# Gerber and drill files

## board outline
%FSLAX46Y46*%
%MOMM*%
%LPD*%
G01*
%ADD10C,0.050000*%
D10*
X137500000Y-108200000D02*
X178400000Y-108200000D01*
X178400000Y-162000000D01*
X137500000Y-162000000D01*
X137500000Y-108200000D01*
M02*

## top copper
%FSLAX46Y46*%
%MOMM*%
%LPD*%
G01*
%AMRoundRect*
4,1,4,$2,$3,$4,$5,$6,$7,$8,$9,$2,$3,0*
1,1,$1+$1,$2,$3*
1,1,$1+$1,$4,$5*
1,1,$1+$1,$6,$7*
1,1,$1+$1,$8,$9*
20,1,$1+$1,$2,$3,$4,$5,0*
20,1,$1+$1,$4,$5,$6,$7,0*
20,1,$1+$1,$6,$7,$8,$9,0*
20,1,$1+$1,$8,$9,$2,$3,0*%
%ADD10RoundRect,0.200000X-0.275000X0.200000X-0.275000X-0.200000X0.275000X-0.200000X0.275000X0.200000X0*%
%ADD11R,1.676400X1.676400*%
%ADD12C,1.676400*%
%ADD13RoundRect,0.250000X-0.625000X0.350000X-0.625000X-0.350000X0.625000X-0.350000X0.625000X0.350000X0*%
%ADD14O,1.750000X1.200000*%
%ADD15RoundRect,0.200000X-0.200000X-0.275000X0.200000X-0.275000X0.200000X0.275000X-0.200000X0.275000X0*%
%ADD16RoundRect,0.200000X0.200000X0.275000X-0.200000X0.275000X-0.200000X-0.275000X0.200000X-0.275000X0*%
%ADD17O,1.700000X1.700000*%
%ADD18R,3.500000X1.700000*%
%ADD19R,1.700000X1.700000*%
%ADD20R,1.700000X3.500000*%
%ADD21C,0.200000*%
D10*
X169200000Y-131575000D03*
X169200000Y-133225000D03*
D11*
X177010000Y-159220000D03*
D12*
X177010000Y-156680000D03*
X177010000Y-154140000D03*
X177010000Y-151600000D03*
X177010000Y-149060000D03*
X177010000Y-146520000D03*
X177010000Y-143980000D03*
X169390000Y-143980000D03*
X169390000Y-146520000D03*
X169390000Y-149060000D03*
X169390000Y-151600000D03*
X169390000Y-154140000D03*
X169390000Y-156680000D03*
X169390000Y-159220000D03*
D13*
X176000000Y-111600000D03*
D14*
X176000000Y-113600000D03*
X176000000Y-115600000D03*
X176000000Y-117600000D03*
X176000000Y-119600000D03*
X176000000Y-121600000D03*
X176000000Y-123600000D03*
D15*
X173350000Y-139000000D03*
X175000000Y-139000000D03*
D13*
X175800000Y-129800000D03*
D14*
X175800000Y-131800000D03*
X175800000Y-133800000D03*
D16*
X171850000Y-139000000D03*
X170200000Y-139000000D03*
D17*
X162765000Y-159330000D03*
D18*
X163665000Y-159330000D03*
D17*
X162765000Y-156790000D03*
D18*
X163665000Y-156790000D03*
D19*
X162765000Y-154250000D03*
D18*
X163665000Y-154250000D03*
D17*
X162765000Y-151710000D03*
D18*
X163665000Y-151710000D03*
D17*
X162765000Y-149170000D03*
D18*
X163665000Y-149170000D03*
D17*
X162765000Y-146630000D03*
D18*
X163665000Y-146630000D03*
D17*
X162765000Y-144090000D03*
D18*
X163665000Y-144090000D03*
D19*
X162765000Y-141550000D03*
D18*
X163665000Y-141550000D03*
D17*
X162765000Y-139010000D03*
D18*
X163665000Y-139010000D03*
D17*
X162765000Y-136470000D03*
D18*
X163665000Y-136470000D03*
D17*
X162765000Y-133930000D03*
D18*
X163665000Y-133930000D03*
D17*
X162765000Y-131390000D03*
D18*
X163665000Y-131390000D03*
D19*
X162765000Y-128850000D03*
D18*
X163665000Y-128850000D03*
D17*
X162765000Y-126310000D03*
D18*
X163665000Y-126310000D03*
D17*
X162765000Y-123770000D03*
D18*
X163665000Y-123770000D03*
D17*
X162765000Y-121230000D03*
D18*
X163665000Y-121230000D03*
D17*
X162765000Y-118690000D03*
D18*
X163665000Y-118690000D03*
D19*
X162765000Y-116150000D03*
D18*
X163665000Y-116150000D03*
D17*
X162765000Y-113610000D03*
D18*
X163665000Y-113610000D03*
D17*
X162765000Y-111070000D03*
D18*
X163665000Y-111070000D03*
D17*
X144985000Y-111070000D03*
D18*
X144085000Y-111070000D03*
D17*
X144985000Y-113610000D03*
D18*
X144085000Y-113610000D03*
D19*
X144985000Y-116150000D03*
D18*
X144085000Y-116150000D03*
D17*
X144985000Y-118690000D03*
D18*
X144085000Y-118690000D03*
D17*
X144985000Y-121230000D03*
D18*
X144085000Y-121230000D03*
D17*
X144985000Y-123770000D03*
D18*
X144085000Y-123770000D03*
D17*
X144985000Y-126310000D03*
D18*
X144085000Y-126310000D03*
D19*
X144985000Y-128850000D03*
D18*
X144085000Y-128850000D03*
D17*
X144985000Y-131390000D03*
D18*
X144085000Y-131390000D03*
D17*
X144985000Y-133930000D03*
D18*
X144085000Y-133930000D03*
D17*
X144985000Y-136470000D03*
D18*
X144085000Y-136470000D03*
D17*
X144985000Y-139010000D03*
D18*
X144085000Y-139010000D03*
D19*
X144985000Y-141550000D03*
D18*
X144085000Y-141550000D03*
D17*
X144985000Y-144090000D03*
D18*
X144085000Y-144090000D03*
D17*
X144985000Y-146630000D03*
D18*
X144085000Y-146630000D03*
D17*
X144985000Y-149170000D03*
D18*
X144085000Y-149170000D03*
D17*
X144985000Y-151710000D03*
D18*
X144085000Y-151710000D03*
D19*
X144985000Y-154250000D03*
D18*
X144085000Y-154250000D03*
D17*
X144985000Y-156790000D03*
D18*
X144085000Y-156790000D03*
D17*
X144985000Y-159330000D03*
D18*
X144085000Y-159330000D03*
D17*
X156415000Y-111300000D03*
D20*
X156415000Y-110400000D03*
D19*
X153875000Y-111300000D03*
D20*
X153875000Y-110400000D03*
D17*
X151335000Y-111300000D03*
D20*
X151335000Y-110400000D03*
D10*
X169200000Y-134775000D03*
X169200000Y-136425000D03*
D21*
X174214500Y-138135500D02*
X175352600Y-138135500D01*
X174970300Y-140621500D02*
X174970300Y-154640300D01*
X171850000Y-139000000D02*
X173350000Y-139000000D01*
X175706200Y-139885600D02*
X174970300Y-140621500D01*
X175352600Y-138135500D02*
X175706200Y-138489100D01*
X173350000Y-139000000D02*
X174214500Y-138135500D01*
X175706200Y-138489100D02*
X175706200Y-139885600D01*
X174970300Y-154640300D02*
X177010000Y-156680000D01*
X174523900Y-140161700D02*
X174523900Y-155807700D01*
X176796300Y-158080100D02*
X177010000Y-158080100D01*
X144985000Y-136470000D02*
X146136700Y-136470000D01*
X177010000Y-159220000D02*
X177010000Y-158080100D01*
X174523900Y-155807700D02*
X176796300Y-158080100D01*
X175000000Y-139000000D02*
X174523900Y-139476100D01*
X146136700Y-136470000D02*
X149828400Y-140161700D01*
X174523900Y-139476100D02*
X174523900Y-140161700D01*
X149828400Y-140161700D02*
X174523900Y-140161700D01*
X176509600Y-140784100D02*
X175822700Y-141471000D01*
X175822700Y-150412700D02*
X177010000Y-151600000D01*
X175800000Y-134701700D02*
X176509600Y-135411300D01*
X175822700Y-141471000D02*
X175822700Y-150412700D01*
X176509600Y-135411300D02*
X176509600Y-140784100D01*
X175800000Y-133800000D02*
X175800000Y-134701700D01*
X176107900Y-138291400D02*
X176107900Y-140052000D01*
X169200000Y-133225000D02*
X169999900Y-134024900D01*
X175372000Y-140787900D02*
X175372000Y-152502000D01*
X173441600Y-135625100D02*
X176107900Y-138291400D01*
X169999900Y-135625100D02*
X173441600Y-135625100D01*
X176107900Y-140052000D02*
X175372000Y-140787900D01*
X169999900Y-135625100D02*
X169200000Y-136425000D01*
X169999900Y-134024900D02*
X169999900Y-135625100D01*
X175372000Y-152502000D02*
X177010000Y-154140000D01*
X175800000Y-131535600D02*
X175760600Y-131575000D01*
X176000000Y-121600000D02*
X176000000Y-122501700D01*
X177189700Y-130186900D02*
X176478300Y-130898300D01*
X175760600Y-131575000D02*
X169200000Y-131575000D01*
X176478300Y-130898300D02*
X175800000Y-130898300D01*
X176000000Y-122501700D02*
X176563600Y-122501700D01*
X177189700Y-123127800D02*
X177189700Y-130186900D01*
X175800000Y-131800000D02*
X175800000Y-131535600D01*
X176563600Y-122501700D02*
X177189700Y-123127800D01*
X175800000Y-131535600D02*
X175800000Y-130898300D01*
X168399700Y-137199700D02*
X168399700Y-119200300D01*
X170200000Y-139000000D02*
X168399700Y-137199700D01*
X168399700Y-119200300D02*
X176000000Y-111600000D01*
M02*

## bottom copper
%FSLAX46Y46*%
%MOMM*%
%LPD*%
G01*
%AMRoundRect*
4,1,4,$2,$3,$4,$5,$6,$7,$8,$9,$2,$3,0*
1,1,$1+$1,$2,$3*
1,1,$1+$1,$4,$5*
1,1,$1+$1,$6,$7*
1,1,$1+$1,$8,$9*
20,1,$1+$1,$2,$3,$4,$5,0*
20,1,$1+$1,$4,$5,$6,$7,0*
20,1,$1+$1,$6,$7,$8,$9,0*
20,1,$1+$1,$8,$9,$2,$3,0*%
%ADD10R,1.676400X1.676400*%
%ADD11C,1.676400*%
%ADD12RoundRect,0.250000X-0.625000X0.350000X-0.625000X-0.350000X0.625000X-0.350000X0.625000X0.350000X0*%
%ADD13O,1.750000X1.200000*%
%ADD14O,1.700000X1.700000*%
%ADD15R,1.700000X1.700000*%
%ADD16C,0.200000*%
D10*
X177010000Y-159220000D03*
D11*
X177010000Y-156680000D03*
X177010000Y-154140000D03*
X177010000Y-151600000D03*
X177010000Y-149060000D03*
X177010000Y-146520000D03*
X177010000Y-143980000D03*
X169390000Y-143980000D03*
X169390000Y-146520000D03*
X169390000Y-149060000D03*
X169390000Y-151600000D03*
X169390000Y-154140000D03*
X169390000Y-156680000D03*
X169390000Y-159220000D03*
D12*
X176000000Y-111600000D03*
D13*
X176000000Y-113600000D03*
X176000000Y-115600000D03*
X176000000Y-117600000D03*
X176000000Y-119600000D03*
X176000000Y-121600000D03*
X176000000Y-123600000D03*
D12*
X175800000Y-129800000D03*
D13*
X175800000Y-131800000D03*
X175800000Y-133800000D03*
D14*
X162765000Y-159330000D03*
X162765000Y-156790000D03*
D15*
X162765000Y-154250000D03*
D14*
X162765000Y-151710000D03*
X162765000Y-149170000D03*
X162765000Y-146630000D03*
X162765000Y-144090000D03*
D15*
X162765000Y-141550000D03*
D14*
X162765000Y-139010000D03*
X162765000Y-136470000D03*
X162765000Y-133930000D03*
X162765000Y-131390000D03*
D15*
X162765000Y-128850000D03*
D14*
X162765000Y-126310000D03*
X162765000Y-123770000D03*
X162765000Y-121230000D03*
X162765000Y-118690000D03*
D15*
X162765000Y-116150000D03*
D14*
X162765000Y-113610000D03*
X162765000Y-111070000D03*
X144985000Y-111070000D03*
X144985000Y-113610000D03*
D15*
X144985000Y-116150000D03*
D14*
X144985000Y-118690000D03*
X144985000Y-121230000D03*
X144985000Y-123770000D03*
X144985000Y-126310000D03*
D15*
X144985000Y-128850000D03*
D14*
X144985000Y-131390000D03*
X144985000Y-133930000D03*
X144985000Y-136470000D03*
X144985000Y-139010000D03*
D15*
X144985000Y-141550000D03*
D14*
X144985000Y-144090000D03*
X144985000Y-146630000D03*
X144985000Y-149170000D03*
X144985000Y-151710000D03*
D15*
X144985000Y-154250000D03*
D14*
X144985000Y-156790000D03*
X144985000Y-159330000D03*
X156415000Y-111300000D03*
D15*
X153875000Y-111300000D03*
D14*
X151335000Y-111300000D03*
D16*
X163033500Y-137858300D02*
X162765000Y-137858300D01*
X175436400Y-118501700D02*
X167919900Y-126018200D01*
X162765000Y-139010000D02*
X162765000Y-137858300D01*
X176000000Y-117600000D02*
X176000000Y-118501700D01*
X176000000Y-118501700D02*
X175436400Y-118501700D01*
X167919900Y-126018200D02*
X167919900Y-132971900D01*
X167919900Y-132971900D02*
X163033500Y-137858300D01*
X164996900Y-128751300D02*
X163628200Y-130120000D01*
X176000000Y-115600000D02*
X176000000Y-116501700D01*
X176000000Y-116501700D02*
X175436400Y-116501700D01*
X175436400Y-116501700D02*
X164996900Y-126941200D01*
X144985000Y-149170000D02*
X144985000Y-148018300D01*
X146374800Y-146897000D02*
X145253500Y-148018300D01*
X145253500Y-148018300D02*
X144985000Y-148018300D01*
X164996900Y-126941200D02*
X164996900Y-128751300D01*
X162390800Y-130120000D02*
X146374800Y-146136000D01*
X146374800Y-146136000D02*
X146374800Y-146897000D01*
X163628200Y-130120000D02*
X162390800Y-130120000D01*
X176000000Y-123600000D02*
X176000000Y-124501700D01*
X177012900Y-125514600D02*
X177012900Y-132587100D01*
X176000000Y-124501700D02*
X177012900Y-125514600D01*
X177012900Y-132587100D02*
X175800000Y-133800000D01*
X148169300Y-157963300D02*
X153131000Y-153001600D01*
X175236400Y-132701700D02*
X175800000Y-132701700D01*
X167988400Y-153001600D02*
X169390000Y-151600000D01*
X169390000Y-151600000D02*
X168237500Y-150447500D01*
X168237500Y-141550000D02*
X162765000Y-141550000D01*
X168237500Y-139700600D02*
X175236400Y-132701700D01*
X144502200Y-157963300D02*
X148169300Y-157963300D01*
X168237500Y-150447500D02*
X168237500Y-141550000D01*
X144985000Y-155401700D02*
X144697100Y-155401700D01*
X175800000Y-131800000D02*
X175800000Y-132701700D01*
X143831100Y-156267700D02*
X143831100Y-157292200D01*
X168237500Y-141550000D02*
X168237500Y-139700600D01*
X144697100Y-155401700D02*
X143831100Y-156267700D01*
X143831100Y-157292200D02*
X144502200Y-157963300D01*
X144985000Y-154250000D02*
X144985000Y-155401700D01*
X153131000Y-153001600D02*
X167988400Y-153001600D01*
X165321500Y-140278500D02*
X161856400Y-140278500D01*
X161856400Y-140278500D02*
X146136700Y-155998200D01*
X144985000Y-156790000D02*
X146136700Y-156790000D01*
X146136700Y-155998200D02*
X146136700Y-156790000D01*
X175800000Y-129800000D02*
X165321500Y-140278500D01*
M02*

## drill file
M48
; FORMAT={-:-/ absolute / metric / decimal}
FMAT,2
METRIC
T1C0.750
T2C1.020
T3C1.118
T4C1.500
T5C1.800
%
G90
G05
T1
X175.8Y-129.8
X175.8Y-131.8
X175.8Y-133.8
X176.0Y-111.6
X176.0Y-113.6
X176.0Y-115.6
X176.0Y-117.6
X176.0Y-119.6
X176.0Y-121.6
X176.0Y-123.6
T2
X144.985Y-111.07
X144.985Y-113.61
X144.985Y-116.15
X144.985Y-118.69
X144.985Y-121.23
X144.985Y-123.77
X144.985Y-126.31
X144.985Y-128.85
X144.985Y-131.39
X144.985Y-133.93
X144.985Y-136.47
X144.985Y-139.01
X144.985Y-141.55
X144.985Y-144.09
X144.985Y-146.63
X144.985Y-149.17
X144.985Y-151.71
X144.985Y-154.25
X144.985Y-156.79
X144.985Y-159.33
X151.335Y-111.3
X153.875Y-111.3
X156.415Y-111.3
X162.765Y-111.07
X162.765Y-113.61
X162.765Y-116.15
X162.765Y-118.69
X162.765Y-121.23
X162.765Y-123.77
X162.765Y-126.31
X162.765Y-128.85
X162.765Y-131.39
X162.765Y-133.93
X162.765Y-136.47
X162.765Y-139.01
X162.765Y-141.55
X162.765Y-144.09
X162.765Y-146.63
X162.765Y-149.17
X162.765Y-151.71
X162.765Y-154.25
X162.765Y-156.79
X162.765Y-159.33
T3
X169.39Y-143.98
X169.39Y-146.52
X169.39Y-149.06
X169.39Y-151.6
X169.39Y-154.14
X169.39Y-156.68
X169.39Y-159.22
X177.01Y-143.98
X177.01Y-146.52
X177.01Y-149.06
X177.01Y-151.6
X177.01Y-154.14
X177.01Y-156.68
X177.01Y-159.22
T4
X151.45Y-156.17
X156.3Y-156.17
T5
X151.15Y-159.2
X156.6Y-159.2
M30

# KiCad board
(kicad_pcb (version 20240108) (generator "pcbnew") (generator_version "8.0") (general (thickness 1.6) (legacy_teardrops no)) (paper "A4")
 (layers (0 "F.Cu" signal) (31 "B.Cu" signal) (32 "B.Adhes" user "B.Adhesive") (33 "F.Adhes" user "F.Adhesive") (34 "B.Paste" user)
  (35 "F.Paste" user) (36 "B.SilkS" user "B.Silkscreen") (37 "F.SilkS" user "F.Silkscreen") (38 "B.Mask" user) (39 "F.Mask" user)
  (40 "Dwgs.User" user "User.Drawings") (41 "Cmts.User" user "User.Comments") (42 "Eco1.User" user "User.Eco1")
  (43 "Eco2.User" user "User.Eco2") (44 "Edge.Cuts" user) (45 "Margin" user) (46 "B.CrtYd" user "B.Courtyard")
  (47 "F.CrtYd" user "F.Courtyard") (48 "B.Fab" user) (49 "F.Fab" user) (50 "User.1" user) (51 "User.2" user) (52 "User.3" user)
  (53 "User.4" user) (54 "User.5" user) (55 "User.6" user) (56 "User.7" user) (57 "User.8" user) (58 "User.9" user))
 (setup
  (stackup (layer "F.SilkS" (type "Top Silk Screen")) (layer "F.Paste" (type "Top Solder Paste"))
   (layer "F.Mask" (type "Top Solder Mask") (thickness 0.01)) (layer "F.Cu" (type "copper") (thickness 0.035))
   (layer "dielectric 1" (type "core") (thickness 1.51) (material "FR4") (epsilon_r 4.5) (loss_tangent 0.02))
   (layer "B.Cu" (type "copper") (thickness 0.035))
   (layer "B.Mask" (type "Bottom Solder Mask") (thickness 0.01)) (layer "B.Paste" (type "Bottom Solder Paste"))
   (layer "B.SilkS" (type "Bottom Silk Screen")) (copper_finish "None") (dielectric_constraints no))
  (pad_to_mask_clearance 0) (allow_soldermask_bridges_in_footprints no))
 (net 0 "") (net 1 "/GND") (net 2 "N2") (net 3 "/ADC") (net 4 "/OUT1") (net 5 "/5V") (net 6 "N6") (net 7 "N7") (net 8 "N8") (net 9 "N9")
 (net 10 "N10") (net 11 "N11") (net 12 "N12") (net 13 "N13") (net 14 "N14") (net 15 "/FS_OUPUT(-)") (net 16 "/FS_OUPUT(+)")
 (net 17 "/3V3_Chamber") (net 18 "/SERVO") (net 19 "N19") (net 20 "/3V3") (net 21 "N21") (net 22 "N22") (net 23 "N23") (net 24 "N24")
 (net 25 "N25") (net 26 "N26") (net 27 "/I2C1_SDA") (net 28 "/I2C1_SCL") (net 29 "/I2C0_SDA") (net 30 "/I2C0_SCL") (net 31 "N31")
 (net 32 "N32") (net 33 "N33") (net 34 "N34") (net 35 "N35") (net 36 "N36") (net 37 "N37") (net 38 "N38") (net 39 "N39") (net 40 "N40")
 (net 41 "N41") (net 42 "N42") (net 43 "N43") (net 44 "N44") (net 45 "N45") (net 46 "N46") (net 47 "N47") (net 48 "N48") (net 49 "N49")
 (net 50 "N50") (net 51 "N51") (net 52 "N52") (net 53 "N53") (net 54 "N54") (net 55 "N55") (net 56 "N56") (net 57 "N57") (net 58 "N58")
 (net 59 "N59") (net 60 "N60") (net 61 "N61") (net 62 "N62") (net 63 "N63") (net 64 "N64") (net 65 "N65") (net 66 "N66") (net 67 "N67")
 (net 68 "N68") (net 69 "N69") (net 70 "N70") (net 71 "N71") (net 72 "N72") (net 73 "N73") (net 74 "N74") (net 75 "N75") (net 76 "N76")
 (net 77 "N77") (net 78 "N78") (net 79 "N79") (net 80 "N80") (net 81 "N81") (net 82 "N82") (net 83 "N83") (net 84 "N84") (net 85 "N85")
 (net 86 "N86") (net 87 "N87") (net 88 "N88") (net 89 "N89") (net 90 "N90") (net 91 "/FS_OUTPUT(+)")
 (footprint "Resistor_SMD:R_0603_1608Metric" (layer "F.Cu") (at 169.2 132.4 -90)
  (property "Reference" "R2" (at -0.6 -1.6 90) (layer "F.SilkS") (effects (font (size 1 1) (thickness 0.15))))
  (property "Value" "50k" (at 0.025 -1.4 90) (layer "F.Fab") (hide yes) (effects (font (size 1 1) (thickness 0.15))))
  (pad "1" smd roundrect (at -0.825 0 270) (size 0.8 0.95) (layers "F.Cu" "F.Paste" "F.Mask") (roundrect_rratio 0.25) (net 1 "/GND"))
  (pad "2" smd roundrect (at 0.825 0 270) (size 0.8 0.95) (layers "F.Cu" "F.Paste" "F.Mask") (roundrect_rratio 0.25) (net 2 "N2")))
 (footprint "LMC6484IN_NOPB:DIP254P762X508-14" (layer "F.Cu") (at 169.39 143.98 180)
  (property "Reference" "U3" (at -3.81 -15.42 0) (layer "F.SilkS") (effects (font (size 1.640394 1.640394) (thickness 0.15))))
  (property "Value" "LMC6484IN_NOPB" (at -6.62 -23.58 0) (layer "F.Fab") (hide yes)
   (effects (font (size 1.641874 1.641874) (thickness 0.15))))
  (pad "1" thru_hole rect (at -7.62 -15.24 180) (size 1.6764 1.6764) (drill 1.1176) (layers "*.Cu" "*.Mask") (remove_unused_layers no)
   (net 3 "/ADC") (solder_mask_margin 0.102))
  (pad "2" thru_hole circle (at -7.62 -12.7 180) (size 1.6764 1.6764) (drill 1.1176) (layers "*.Cu" "*.Mask") (remove_unused_layers no)
   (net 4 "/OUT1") (solder_mask_margin 0.102))
  (pad "3" thru_hole circle (at -7.62 -10.16 180) (size 1.6764 1.6764) (drill 1.1176) (layers "*.Cu" "*.Mask") (remove_unused_layers no)
   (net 2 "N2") (solder_mask_margin 0.102))
  (pad "4" thru_hole circle (at -7.62 -7.62 180) (size 1.6764 1.6764) (drill 1.1176) (layers "*.Cu" "*.Mask") (remove_unused_layers no)
   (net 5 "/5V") (solder_mask_margin 0.102))
  (pad "5" thru_hole circle (at -7.62 -5.08 180) (size 1.6764 1.6764) (drill 1.1176) (layers "*.Cu" "*.Mask") (remove_unused_layers no)
   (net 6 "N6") (solder_mask_margin 0.102))
  (pad "6" thru_hole circle (at -7.62 -2.54 180) (size 1.6764 1.6764) (drill 1.1176) (layers "*.Cu" "*.Mask") (remove_unused_layers no)
   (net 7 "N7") (solder_mask_margin 0.102))
  (pad "7" thru_hole circle (at -7.62 0 180) (size 1.6764 1.6764) (drill 1.1176) (layers "*.Cu" "*.Mask") (remove_unused_layers no)
   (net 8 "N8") (solder_mask_margin 0.102))
  (pad "8" thru_hole circle (at 0 0 180) (size 1.6764 1.6764) (drill 1.1176) (layers "*.Cu" "*.Mask") (remove_unused_layers no) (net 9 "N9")
   (solder_mask_margin 0.102))
  (pad "9" thru_hole circle (at 0 -2.54 180) (size 1.6764 1.6764) (drill 1.1176) (layers "*.Cu" "*.Mask") (remove_unused_layers no)
   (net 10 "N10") (solder_mask_margin 0.102))
  (pad "10" thru_hole circle (at 0 -5.08 180) (size 1.6764 1.6764) (drill 1.1176) (layers "*.Cu" "*.Mask") (remove_unused_layers no)
   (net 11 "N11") (solder_mask_margin 0.102))
  (pad "11" thru_hole circle (at 0 -7.62 180) (size 1.6764 1.6764) (drill 1.1176) (layers "*.Cu" "*.Mask") (remove_unused_layers no)
   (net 1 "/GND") (solder_mask_margin 0.102))
  (pad "12" thru_hole circle (at 0 -10.16 180) (size 1.6764 1.6764) (drill 1.1176) (layers "*.Cu" "*.Mask") (remove_unused_layers no)
   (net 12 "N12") (solder_mask_margin 0.102))
  (pad "13" thru_hole circle (at 0 -12.7 180) (size 1.6764 1.6764) (drill 1.1176) (layers "*.Cu" "*.Mask") (remove_unused_layers no)
   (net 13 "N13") (solder_mask_margin 0.102))
  (pad "14" thru_hole circle (at 0 -15.24 180) (size 1.6764 1.6764) (drill 1.1176) (layers "*.Cu" "*.Mask") (remove_unused_layers no)
   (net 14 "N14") (solder_mask_margin 0.102)))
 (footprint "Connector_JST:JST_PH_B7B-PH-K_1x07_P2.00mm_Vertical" (layer "F.Cu") (at 176 111.6 -90)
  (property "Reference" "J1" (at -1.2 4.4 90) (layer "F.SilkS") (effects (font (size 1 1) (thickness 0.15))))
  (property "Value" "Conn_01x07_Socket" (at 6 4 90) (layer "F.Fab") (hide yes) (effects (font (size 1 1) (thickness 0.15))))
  (pad "1" thru_hole roundrect (at 0 0 270) (size 1.2 1.75) (drill 0.75) (layers "*.Cu" "*.Mask") (remove_unused_layers no)
   (roundrect_rratio 0.208333) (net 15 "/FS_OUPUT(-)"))
  (pad "2" thru_hole oval (at 2 0 270) (size 1.2 1.75) (drill 0.75) (layers "*.Cu" "*.Mask") (remove_unused_layers no)
   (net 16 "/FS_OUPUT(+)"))
  (pad "3" thru_hole oval (at 4 0 270) (size 1.2 1.75) (drill 0.75) (layers "*.Cu" "*.Mask") (remove_unused_layers no)
   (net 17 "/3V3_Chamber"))
  (pad "4" thru_hole oval (at 6 0 270) (size 1.2 1.75) (drill 0.75) (layers "*.Cu" "*.Mask") (remove_unused_layers no) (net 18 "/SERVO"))
  (pad "5" thru_hole oval (at 8 0 270) (size 1.2 1.75) (drill 0.75) (layers "*.Cu" "*.Mask") (remove_unused_layers no) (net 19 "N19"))
  (pad "6" thru_hole oval (at 10 0 270) (size 1.2 1.75) (drill 0.75) (layers "*.Cu" "*.Mask") (remove_unused_layers no) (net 1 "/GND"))
  (pad "7" thru_hole oval (at 12 0 270) (size 1.2 1.75) (drill 0.75) (layers "*.Cu" "*.Mask") (remove_unused_layers no) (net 5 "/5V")))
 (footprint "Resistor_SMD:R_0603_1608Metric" (layer "F.Cu") (at 174.175 139)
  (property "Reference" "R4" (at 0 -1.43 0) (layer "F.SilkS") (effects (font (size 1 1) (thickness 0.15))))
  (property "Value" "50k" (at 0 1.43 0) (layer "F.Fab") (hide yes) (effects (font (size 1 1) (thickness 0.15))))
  (pad "1" smd roundrect (at -0.825 0) (size 0.8 0.95) (layers "F.Cu" "F.Paste" "F.Mask") (roundrect_rratio 0.25) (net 4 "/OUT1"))
  (pad "2" smd roundrect (at 0.825 0) (size 0.8 0.95) (layers "F.Cu" "F.Paste" "F.Mask") (roundrect_rratio 0.25) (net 3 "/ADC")))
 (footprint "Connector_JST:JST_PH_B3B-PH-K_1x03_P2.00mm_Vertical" (layer "F.Cu") (at 175.8 129.8 -90)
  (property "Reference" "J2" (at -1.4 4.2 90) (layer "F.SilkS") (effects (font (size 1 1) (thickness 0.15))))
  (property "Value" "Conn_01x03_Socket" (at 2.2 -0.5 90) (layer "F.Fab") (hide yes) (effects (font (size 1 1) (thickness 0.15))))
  (pad "1" thru_hole roundrect (at 0 0 270) (size 1.2 1.75) (drill 0.75) (layers "*.Cu" "*.Mask") (remove_unused_layers no)
   (roundrect_rratio 0.208333) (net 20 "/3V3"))
  (pad "2" thru_hole oval (at 2 0 270) (size 1.2 1.75) (drill 0.75) (layers "*.Cu" "*.Mask") (remove_unused_layers no) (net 1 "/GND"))
  (pad "3" thru_hole oval (at 4 0 270) (size 1.2 1.75) (drill 0.75) (layers "*.Cu" "*.Mask") (remove_unused_layers no) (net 5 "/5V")))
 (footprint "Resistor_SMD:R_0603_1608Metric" (layer "F.Cu") (at 171.025 139 180)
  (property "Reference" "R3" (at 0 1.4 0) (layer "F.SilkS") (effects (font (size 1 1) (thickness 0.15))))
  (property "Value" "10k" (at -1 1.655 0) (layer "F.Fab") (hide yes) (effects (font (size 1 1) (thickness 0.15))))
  (pad "1" smd roundrect (at -0.825 0 180) (size 0.8 0.95) (layers "F.Cu" "F.Paste" "F.Mask") (roundrect_rratio 0.25) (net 4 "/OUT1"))
  (pad "2" smd roundrect (at 0.825 0 180) (size 0.8 0.95) (layers "F.Cu" "F.Paste" "F.Mask") (roundrect_rratio 0.25) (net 15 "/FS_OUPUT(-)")))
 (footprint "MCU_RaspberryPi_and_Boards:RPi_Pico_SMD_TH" (layer "F.Cu") (at 153.875 135.2 180)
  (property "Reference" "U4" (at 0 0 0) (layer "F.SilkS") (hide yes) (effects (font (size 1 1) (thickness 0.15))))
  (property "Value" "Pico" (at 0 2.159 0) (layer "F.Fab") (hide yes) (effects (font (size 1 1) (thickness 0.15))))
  (pad "" np_thru_hole oval (at -2.725 -24 180) (size 1.8 1.8) (drill 1.8) (layers "*.Cu" "*.Mask"))
  (pad "" np_thru_hole oval (at -2.425 -20.97 180) (size 1.5 1.5) (drill 1.5) (layers "*.Cu" "*.Mask"))
  (pad "" np_thru_hole oval (at 2.425 -20.97 180) (size 1.5 1.5) (drill 1.5) (layers "*.Cu" "*.Mask"))
  (pad "" np_thru_hole oval (at 2.725 -24 180) (size 1.8 1.8) (drill 1.8) (layers "*.Cu" "*.Mask"))
  (pad "1" thru_hole oval (at -8.89 -24.13 180) (size 1.7 1.7) (drill 1.02) (layers "*.Cu" "*.Mask") (remove_unused_layers no)
   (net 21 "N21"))
  (pad "1" smd rect (at -8.89 -24.13 180) (size 3.5 1.7) (drill (offset -0.9 0)) (layers "F.Cu" "F.Mask") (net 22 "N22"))
  (pad "2" thru_hole oval (at -8.89 -21.59 180) (size 1.7 1.7) (drill 1.02) (layers "*.Cu" "*.Mask") (remove_unused_layers no)
   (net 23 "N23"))
  (pad "2" smd rect (at -8.89 -21.59 180) (size 3.5 1.7) (drill (offset -0.9 0)) (layers "F.Cu" "F.Mask") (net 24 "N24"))
  (pad "3" thru_hole rect (at -8.89 -19.05 180) (size 1.7 1.7) (drill 1.02) (layers "*.Cu" "*.Mask") (remove_unused_layers no)
   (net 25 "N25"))
  (pad "3" smd rect (at -8.89 -19.05 180) (size 3.5 1.7) (drill (offset -0.9 0)) (layers "F.Cu" "F.Mask") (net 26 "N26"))
  (pad "4" thru_hole oval (at -8.89 -16.51 180) (size 1.7 1.7) (drill 1.02) (layers "*.Cu" "*.Mask") (remove_unused_layers no)
   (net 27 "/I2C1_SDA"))
  (pad "4" smd rect (at -8.89 -16.51 180) (size 3.5 1.7) (drill (offset -0.9 0)) (layers "F.Cu" "F.Mask") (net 27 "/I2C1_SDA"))
  (pad "5" thru_hole oval (at -8.89 -13.97 180) (size 1.7 1.7) (drill 1.02) (layers "*.Cu" "*.Mask") (remove_unused_layers no)
   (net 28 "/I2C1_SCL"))
  (pad "5" smd rect (at -8.89 -13.97 180) (size 3.5 1.7) (drill (offset -0.9 0)) (layers "F.Cu" "F.Mask") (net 28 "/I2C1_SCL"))
  (pad "6" thru_hole oval (at -8.89 -11.43 180) (size 1.7 1.7) (drill 1.02) (layers "*.Cu" "*.Mask") (remove_unused_layers no)
   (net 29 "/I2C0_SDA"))
  (pad "6" smd rect (at -8.89 -11.43 180) (size 3.5 1.7) (drill (offset -0.9 0)) (layers "F.Cu" "F.Mask") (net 29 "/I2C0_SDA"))
  (pad "7" thru_hole oval (at -8.89 -8.89 180) (size 1.7 1.7) (drill 1.02) (layers "*.Cu" "*.Mask") (remove_unused_layers no)
   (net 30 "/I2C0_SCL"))
  (pad "7" smd rect (at -8.89 -8.89 180) (size 3.5 1.7) (drill (offset -0.9 0)) (layers "F.Cu" "F.Mask") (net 30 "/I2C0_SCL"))
  (pad "8" thru_hole rect (at -8.89 -6.35 180) (size 1.7 1.7) (drill 1.02) (layers "*.Cu" "*.Mask") (remove_unused_layers no) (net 1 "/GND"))
  (pad "8" smd rect (at -8.89 -6.35 180) (size 3.5 1.7) (drill (offset -0.9 0)) (layers "F.Cu" "F.Mask") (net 1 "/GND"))
  (pad "9" thru_hole oval (at -8.89 -3.81 180) (size 1.7 1.7) (drill 1.02) (layers "*.Cu" "*.Mask") (remove_unused_layers no)
   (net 18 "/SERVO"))
  (pad "9" smd rect (at -8.89 -3.81 180) (size 3.5 1.7) (drill (offset -0.9 0)) (layers "F.Cu" "F.Mask") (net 18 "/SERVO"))
  (pad "10" thru_hole oval (at -8.89 -1.27 180) (size 1.7 1.7) (drill 1.02) (layers "*.Cu" "*.Mask") (remove_unused_layers no)
   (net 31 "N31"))
  (pad "10" smd rect (at -8.89 -1.27 180) (size 3.5 1.7) (drill (offset -0.9 0)) (layers "F.Cu" "F.Mask") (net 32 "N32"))
  (pad "11" thru_hole oval (at -8.89 1.27 180) (size 1.7 1.7) (drill 1.02) (layers "*.Cu" "*.Mask") (remove_unused_layers no) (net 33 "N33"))
  (pad "11" smd rect (at -8.89 1.27 180) (size 3.5 1.7) (drill (offset -0.9 0)) (layers "F.Cu" "F.Mask") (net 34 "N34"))
  (pad "12" thru_hole oval (at -8.89 3.81 180) (size 1.7 1.7) (drill 1.02) (layers "*.Cu" "*.Mask") (remove_unused_layers no) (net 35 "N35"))
  (pad "12" smd rect (at -8.89 3.81 180) (size 3.5 1.7) (drill (offset -0.9 0)) (layers "F.Cu" "F.Mask") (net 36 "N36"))
  (pad "13" thru_hole rect (at -8.89 6.35 180) (size 1.7 1.7) (drill 1.02) (layers "*.Cu" "*.Mask") (remove_unused_layers no) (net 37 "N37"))
  (pad "13" smd rect (at -8.89 6.35 180) (size 3.5 1.7) (drill (offset -0.9 0)) (layers "F.Cu" "F.Mask") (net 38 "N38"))
  (pad "14" thru_hole oval (at -8.89 8.89 180) (size 1.7 1.7) (drill 1.02) (layers "*.Cu" "*.Mask") (remove_unused_layers no) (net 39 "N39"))
  (pad "14" smd rect (at -8.89 8.89 180) (size 3.5 1.7) (drill (offset -0.9 0)) (layers "F.Cu" "F.Mask") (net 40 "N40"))
  (pad "15" thru_hole oval (at -8.89 11.43 180) (size 1.7 1.7) (drill 1.02) (layers "*.Cu" "*.Mask") (remove_unused_layers no)
   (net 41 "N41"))
  (pad "15" smd rect (at -8.89 11.43 180) (size 3.5 1.7) (drill (offset -0.9 0)) (layers "F.Cu" "F.Mask") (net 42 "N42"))
  (pad "16" thru_hole oval (at -8.89 13.97 180) (size 1.7 1.7) (drill 1.02) (layers "*.Cu" "*.Mask") (remove_unused_layers no)
   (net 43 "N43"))
  (pad "16" smd rect (at -8.89 13.97 180) (size 3.5 1.7) (drill (offset -0.9 0)) (layers "F.Cu" "F.Mask") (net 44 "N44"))
  (pad "17" thru_hole oval (at -8.89 16.51 180) (size 1.7 1.7) (drill 1.02) (layers "*.Cu" "*.Mask") (remove_unused_layers no)
   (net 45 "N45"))
  (pad "17" smd rect (at -8.89 16.51 180) (size 3.5 1.7) (drill (offset -0.9 0)) (layers "F.Cu" "F.Mask") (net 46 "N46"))
  (pad "18" thru_hole rect (at -8.89 19.05 180) (size 1.7 1.7) (drill 1.02) (layers "*.Cu" "*.Mask") (remove_unused_layers no)
   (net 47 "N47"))
  (pad "18" smd rect (at -8.89 19.05 180) (size 3.5 1.7) (drill (offset -0.9 0)) (layers "F.Cu" "F.Mask") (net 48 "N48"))
  (pad "19" thru_hole oval (at -8.89 21.59 180) (size 1.7 1.7) (drill 1.02) (layers "*.Cu" "*.Mask") (remove_unused_layers no)
   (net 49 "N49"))
  (pad "19" smd rect (at -8.89 21.59 180) (size 3.5 1.7) (drill (offset -0.9 0)) (layers "F.Cu" "F.Mask") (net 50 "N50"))
  (pad "20" thru_hole oval (at -8.89 24.13 180) (size 1.7 1.7) (drill 1.02) (layers "*.Cu" "*.Mask") (remove_unused_layers no)
   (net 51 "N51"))
  (pad "20" smd rect (at -8.89 24.13 180) (size 3.5 1.7) (drill (offset -0.9 0)) (layers "F.Cu" "F.Mask") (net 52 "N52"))
  (pad "21" thru_hole oval (at 8.89 24.13 180) (size 1.7 1.7) (drill 1.02) (layers "*.Cu" "*.Mask") (remove_unused_layers no) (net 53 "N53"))
  (pad "21" smd rect (at 8.89 24.13 180) (size 3.5 1.7) (drill (offset 0.9 0)) (layers "F.Cu" "F.Mask") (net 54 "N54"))
  (pad "22" thru_hole oval (at 8.89 21.59 180) (size 1.7 1.7) (drill 1.02) (layers "*.Cu" "*.Mask") (remove_unused_layers no) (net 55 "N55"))
  (pad "22" smd rect (at 8.89 21.59 180) (size 3.5 1.7) (drill (offset 0.9 0)) (layers "F.Cu" "F.Mask") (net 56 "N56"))
  (pad "23" thru_hole rect (at 8.89 19.05 180) (size 1.7 1.7) (drill 1.02) (layers "*.Cu" "*.Mask") (remove_unused_layers no) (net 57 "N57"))
  (pad "23" smd rect (at 8.89 19.05 180) (size 3.5 1.7) (drill (offset 0.9 0)) (layers "F.Cu" "F.Mask") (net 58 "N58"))
  (pad "24" thru_hole oval (at 8.89 16.51 180) (size 1.7 1.7) (drill 1.02) (layers "*.Cu" "*.Mask") (remove_unused_layers no) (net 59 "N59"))
  (pad "24" smd rect (at 8.89 16.51 180) (size 3.5 1.7) (drill (offset 0.9 0)) (layers "F.Cu" "F.Mask") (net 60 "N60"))
  (pad "25" thru_hole oval (at 8.89 13.97 180) (size 1.7 1.7) (drill 1.02) (layers "*.Cu" "*.Mask") (remove_unused_layers no) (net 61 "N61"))
  (pad "25" smd rect (at 8.89 13.97 180) (size 3.5 1.7) (drill (offset 0.9 0)) (layers "F.Cu" "F.Mask") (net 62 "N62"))
  (pad "26" thru_hole oval (at 8.89 11.43 180) (size 1.7 1.7) (drill 1.02) (layers "*.Cu" "*.Mask") (remove_unused_layers no) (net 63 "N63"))
  (pad "26" smd rect (at 8.89 11.43 180) (size 3.5 1.7) (drill (offset 0.9 0)) (layers "F.Cu" "F.Mask") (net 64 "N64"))
  (pad "27" thru_hole oval (at 8.89 8.89 180) (size 1.7 1.7) (drill 1.02) (layers "*.Cu" "*.Mask") (remove_unused_layers no) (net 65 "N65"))
  (pad "27" smd rect (at 8.89 8.89 180) (size 3.5 1.7) (drill (offset 0.9 0)) (layers "F.Cu" "F.Mask") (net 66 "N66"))
  (pad "28" thru_hole rect (at 8.89 6.35 180) (size 1.7 1.7) (drill 1.02) (layers "*.Cu" "*.Mask") (remove_unused_layers no) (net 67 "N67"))
  (pad "28" smd rect (at 8.89 6.35 180) (size 3.5 1.7) (drill (offset 0.9 0)) (layers "F.Cu" "F.Mask") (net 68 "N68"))
  (pad "29" thru_hole oval (at 8.89 3.81 180) (size 1.7 1.7) (drill 1.02) (layers "*.Cu" "*.Mask") (remove_unused_layers no) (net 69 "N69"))
  (pad "29" smd rect (at 8.89 3.81 180) (size 3.5 1.7) (drill (offset 0.9 0)) (layers "F.Cu" "F.Mask") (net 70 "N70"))
  (pad "30" thru_hole oval (at 8.89 1.27 180) (size 1.7 1.7) (drill 1.02) (layers "*.Cu" "*.Mask") (remove_unused_layers no) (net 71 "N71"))
  (pad "30" smd rect (at 8.89 1.27 180) (size 3.5 1.7) (drill (offset 0.9 0)) (layers "F.Cu" "F.Mask") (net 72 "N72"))
  (pad "31" thru_hole oval (at 8.89 -1.27 180) (size 1.7 1.7) (drill 1.02) (layers "*.Cu" "*.Mask") (remove_unused_layers no) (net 3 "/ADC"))
  (pad "31" smd rect (at 8.89 -1.27 180) (size 3.5 1.7) (drill (offset 0.9 0)) (layers "F.Cu" "F.Mask") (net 3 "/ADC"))
  (pad "32" thru_hole oval (at 8.89 -3.81 180) (size 1.7 1.7) (drill 1.02) (layers "*.Cu" "*.Mask") (remove_unused_layers no) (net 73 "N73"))
  (pad "32" smd rect (at 8.89 -3.81 180) (size 3.5 1.7) (drill (offset 0.9 0)) (layers "F.Cu" "F.Mask") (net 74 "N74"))
  (pad "33" thru_hole rect (at 8.89 -6.35 180) (size 1.7 1.7) (drill 1.02) (layers "*.Cu" "*.Mask") (remove_unused_layers no) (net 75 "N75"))
  (pad "33" smd rect (at 8.89 -6.35 180) (size 3.5 1.7) (drill (offset 0.9 0)) (layers "F.Cu" "F.Mask") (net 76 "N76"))
  (pad "34" thru_hole oval (at 8.89 -8.89 180) (size 1.7 1.7) (drill 1.02) (layers "*.Cu" "*.Mask") (remove_unused_layers no) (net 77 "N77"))
  (pad "34" smd rect (at 8.89 -8.89 180) (size 3.5 1.7) (drill (offset 0.9 0)) (layers "F.Cu" "F.Mask") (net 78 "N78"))
  (pad "35" thru_hole oval (at 8.89 -11.43 180) (size 1.7 1.7) (drill 1.02) (layers "*.Cu" "*.Mask") (remove_unused_layers no)
   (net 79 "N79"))
  (pad "35" smd rect (at 8.89 -11.43 180) (size 3.5 1.7) (drill (offset 0.9 0)) (layers "F.Cu" "F.Mask") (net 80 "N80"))
  (pad "36" thru_hole oval (at 8.89 -13.97 180) (size 1.7 1.7) (drill 1.02) (layers "*.Cu" "*.Mask") (remove_unused_layers no)
   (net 17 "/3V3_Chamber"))
  (pad "36" smd rect (at 8.89 -13.97 180) (size 3.5 1.7) (drill (offset 0.9 0)) (layers "F.Cu" "F.Mask") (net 17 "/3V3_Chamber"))
  (pad "37" thru_hole oval (at 8.89 -16.51 180) (size 1.7 1.7) (drill 1.02) (layers "*.Cu" "*.Mask") (remove_unused_layers no)
   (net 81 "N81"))
  (pad "37" smd rect (at 8.89 -16.51 180) (size 3.5 1.7) (drill (offset 0.9 0)) (layers "F.Cu" "F.Mask") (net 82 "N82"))
  (pad "38" thru_hole rect (at 8.89 -19.05 180) (size 1.7 1.7) (drill 1.02) (layers "*.Cu" "*.Mask") (remove_unused_layers no)
   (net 1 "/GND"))
  (pad "38" smd rect (at 8.89 -19.05 180) (size 3.5 1.7) (drill (offset 0.9 0)) (layers "F.Cu" "F.Mask") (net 1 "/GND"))
  (pad "39" thru_hole oval (at 8.89 -21.59 180) (size 1.7 1.7) (drill 1.02) (layers "*.Cu" "*.Mask") (remove_unused_layers no)
   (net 20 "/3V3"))
  (pad "39" smd rect (at 8.89 -21.59 180) (size 3.5 1.7) (drill (offset 0.9 0)) (layers "F.Cu" "F.Mask") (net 20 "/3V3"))
  (pad "40" thru_hole oval (at 8.89 -24.13 180) (size 1.7 1.7) (drill 1.02) (layers "*.Cu" "*.Mask") (remove_unused_layers no)
   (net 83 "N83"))
  (pad "40" smd rect (at 8.89 -24.13 180) (size 3.5 1.7) (drill (offset 0.9 0)) (layers "F.Cu" "F.Mask") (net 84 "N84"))
  (pad "41" thru_hole oval (at -2.54 23.9 180) (size 1.7 1.7) (drill 1.02) (layers "*.Cu" "*.Mask") (remove_unused_layers no) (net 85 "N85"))
  (pad "41" smd rect (at -2.54 23.9 270) (size 3.5 1.7) (drill (offset -0.9 0)) (layers "F.Cu" "F.Mask") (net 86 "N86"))
  (pad "42" thru_hole rect (at 0 23.9 180) (size 1.7 1.7) (drill 1.02) (layers "*.Cu" "*.Mask") (remove_unused_layers no) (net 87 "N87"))
  (pad "42" smd rect (at 0 23.9 270) (size 3.5 1.7) (drill (offset -0.9 0)) (layers "F.Cu" "F.Mask") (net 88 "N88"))
  (pad "43" thru_hole oval (at 2.54 23.9 180) (size 1.7 1.7) (drill 1.02) (layers "*.Cu" "*.Mask") (remove_unused_layers no) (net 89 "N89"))
  (pad "43" smd rect (at 2.54 23.9 270) (size 3.5 1.7) (drill (offset -0.9 0)) (layers "F.Cu" "F.Mask") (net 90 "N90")))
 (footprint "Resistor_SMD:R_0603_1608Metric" (layer "F.Cu") (at 169.2 135.6 -90)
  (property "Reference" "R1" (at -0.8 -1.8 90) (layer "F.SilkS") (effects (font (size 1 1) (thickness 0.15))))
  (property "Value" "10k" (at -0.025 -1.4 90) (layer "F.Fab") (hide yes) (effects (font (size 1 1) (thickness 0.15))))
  (pad "1" smd roundrect (at -0.825 0 270) (size 0.8 0.95) (layers "F.Cu" "F.Paste" "F.Mask") (roundrect_rratio 0.25)
   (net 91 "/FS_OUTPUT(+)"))
  (pad "2" smd roundrect (at 0.825 0 270) (size 0.8 0.95) (layers "F.Cu" "F.Paste" "F.Mask") (roundrect_rratio 0.25) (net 2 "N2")))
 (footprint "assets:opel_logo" (layer "B.Cu") (at 154 122.4 180)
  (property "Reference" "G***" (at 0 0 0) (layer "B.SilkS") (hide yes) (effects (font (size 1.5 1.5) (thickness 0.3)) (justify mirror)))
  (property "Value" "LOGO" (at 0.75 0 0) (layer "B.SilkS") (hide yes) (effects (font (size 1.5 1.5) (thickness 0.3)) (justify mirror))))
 (gr_rect (start 137.5 108.2) (end 178.4 162) (stroke (width 0.05) (type default)) (fill none) (layer "Edge.Cuts"))
 (segment (start 163.0335 137.8583) (end 162.765 137.8583) (width 0.2) (layer "B.Cu") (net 18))
 (segment (start 175.4364 118.5017) (end 167.9199 126.0182) (width 0.2) (layer "B.Cu") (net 18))
 (segment (start 162.765 139.01) (end 162.765 137.8583) (width 0.2) (layer "B.Cu") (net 18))
 (segment (start 176 117.6) (end 176 118.5017) (width 0.2) (layer "B.Cu") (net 18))
 (segment (start 176 118.5017) (end 175.4364 118.5017) (width 0.2) (layer "B.Cu") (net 18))
 (segment (start 167.9199 126.0182) (end 167.9199 132.9719) (width 0.2) (layer "B.Cu") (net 18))
 (segment (start 167.9199 132.9719) (end 163.0335 137.8583) (width 0.2) (layer "B.Cu") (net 18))
 (segment (start 164.9969 128.7513) (end 163.6282 130.12) (width 0.2) (layer "B.Cu") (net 17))
 (segment (start 176 115.6) (end 176 116.5017) (width 0.2) (layer "B.Cu") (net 17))
 (segment (start 176 116.5017) (end 175.4364 116.5017) (width 0.2) (layer "B.Cu") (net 17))
 (segment (start 175.4364 116.5017) (end 164.9969 126.9412) (width 0.2) (layer "B.Cu") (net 17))
 (segment (start 144.985 149.17) (end 144.985 148.0183) (width 0.2) (layer "B.Cu") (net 17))
 (segment (start 146.3748 146.897) (end 145.2535 148.0183) (width 0.2) (layer "B.Cu") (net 17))
 (segment (start 145.2535 148.0183) (end 144.985 148.0183) (width 0.2) (layer "B.Cu") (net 17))
 (segment (start 164.9969 126.9412) (end 164.9969 128.7513) (width 0.2) (layer "B.Cu") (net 17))
 (segment (start 162.3908 130.12) (end 146.3748 146.136) (width 0.2) (layer "B.Cu") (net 17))
 (segment (start 146.3748 146.136) (end 146.3748 146.897) (width 0.2) (layer "B.Cu") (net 17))
 (segment (start 163.6282 130.12) (end 162.3908 130.12) (width 0.2) (layer "B.Cu") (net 17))
 (segment (start 174.2145 138.1355) (end 175.3526 138.1355) (width 0.2) (layer "F.Cu") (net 4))
 (segment (start 174.9703 140.6215) (end 174.9703 154.6403) (width 0.2) (layer "F.Cu") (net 4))
 (segment (start 171.85 139) (end 173.35 139) (width 0.2) (layer "F.Cu") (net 4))
 (segment (start 175.7062 139.8856) (end 174.9703 140.6215) (width 0.2) (layer "F.Cu") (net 4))
 (segment (start 175.3526 138.1355) (end 175.7062 138.4891) (width 0.2) (layer "F.Cu") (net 4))
 (segment (start 173.35 139) (end 174.2145 138.1355) (width 0.2) (layer "F.Cu") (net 4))
 (segment (start 175.7062 138.4891) (end 175.7062 139.8856) (width 0.2) (layer "F.Cu") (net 4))
 (segment (start 174.9703 154.6403) (end 177.01 156.68) (width 0.2) (layer "F.Cu") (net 4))
 (segment (start 174.5239 140.1617) (end 174.5239 155.8077) (width 0.2) (layer "F.Cu") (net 3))
 (segment (start 176.7963 158.0801) (end 177.01 158.0801) (width 0.2) (layer "F.Cu") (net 3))
 (segment (start 144.985 136.47) (end 146.1367 136.47) (width 0.2) (layer "F.Cu") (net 3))
 (segment (start 177.01 159.22) (end 177.01 158.0801) (width 0.2) (layer "F.Cu") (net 3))
 (segment (start 174.5239 155.8077) (end 176.7963 158.0801) (width 0.2) (layer "F.Cu") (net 3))
 (segment (start 175 139) (end 174.5239 139.4761) (width 0.2) (layer "F.Cu") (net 3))
 (segment (start 146.1367 136.47) (end 149.8284 140.1617) (width 0.2) (layer "F.Cu") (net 3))
 (segment (start 174.5239 139.4761) (end 174.5239 140.1617) (width 0.2) (layer "F.Cu") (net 3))
 (segment (start 149.8284 140.1617) (end 174.5239 140.1617) (width 0.2) (layer "F.Cu") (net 3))
 (segment (start 176.5096 140.7841) (end 175.8227 141.471) (width 0.2) (layer "F.Cu") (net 5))
 (segment (start 175.8227 150.4127) (end 177.01 151.6) (width 0.2) (layer "F.Cu") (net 5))
 (segment (start 175.8 134.7017) (end 176.5096 135.4113) (width 0.2) (layer "F.Cu") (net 5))
 (segment (start 175.8227 141.471) (end 175.8227 150.4127) (width 0.2) (layer "F.Cu") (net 5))
 (segment (start 176.5096 135.4113) (end 176.5096 140.7841) (width 0.2) (layer "F.Cu") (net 5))
 (segment (start 175.8 133.8) (end 175.8 134.7017) (width 0.2) (layer "F.Cu") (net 5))
 (segment (start 176 123.6) (end 176 124.5017) (width 0.2) (layer "B.Cu") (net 5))
 (segment (start 177.0129 125.5146) (end 177.0129 132.5871) (width 0.2) (layer "B.Cu") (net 5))
 (segment (start 176 124.5017) (end 177.0129 125.5146) (width 0.2) (layer "B.Cu") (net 5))
 (segment (start 177.0129 132.5871) (end 175.8 133.8) (width 0.2) (layer "B.Cu") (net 5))
 (segment (start 176.1079 138.2914) (end 176.1079 140.052) (width 0.2) (layer "F.Cu") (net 2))
 (segment (start 169.2 133.225) (end 169.9999 134.0249) (width 0.2) (layer "F.Cu") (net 2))
 (segment (start 175.372 140.7879) (end 175.372 152.502) (width 0.2) (layer "F.Cu") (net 2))
 (segment (start 173.4416 135.6251) (end 176.1079 138.2914) (width 0.2) (layer "F.Cu") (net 2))
 (segment (start 169.9999 135.6251) (end 173.4416 135.6251) (width 0.2) (layer "F.Cu") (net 2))
 (segment (start 176.1079 140.052) (end 175.372 140.7879) (width 0.2) (layer "F.Cu") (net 2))
 (segment (start 169.9999 135.6251) (end 169.2 136.425) (width 0.2) (layer "F.Cu") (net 2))
 (segment (start 169.9999 134.0249) (end 169.9999 135.6251) (width 0.2) (layer "F.Cu") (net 2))
 (segment (start 175.372 152.502) (end 177.01 154.14) (width 0.2) (layer "F.Cu") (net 2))
 (segment (start 175.8 131.5356) (end 175.7606 131.575) (width 0.2) (layer "F.Cu") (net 1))
 (segment (start 176 121.6) (end 176 122.5017) (width 0.2) (layer "F.Cu") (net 1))
 (segment (start 177.1897 130.1869) (end 176.4783 130.8983) (width 0.2) (layer "F.Cu") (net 1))
 (segment (start 175.7606 131.575) (end 169.2 131.575) (width 0.2) (layer "F.Cu") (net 1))
 (segment (start 176.4783 130.8983) (end 175.8 130.8983) (width 0.2) (layer "F.Cu") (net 1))
 (segment (start 176 122.5017) (end 176.5636 122.5017) (width 0.2) (layer "F.Cu") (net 1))
 (segment (start 177.1897 123.1278) (end 177.1897 130.1869) (width 0.2) (layer "F.Cu") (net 1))
 (segment (start 175.8 131.8) (end 175.8 131.5356) (width 0.2) (layer "F.Cu") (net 1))
 (segment (start 176.5636 122.5017) (end 177.1897 123.1278) (width 0.2) (layer "F.Cu") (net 1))
 (segment (start 175.8 131.5356) (end 175.8 130.8983) (width 0.2) (layer "F.Cu") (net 1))
 (segment (start 148.1693 157.9633) (end 153.131 153.0016) (width 0.2) (layer "B.Cu") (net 1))
 (segment (start 175.2364 132.7017) (end 175.8 132.7017) (width 0.2) (layer "B.Cu") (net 1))
 (segment (start 167.9884 153.0016) (end 169.39 151.6) (width 0.2) (layer "B.Cu") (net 1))
 (segment (start 169.39 151.6) (end 168.2375 150.4475) (width 0.2) (layer "B.Cu") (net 1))
 (segment (start 168.2375 141.55) (end 162.765 141.55) (width 0.2) (layer "B.Cu") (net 1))
 (segment (start 168.2375 139.7006) (end 175.2364 132.7017) (width 0.2) (layer "B.Cu") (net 1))
 (segment (start 144.5022 157.9633) (end 148.1693 157.9633) (width 0.2) (layer "B.Cu") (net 1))
 (segment (start 168.2375 150.4475) (end 168.2375 141.55) (width 0.2) (layer "B.Cu") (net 1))
 (segment (start 144.985 155.4017) (end 144.6971 155.4017) (width 0.2) (layer "B.Cu") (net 1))
 (segment (start 175.8 131.8) (end 175.8 132.7017) (width 0.2) (layer "B.Cu") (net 1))
 (segment (start 143.8311 156.2677) (end 143.8311 157.2922) (width 0.2) (layer "B.Cu") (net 1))
 (segment (start 168.2375 141.55) (end 168.2375 139.7006) (width 0.2) (layer "B.Cu") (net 1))
 (segment (start 144.6971 155.4017) (end 143.8311 156.2677) (width 0.2) (layer "B.Cu") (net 1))
 (segment (start 143.8311 157.2922) (end 144.5022 157.9633) (width 0.2) (layer "B.Cu") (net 1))
 (segment (start 144.985 154.25) (end 144.985 155.4017) (width 0.2) (layer "B.Cu") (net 1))
 (segment (start 153.131 153.0016) (end 167.9884 153.0016) (width 0.2) (layer "B.Cu") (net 1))
 (segment (start 165.3215 140.2785) (end 161.8564 140.2785) (width 0.2) (layer "B.Cu") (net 20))
 (segment (start 161.8564 140.2785) (end 146.1367 155.9982) (width 0.2) (layer "B.Cu") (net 20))
 (segment (start 144.985 156.79) (end 146.1367 156.79) (width 0.2) (layer "B.Cu") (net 20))
 (segment (start 146.1367 155.9982) (end 146.1367 156.79) (width 0.2) (layer "B.Cu") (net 20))
 (segment (start 175.8 129.8) (end 165.3215 140.2785) (width 0.2) (layer "B.Cu") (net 20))
 (segment (start 168.3997 137.1997) (end 168.3997 119.2003) (width 0.2) (layer "F.Cu") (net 15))
 (segment (start 170.2 139) (end 168.3997 137.1997) (width 0.2) (layer "F.Cu") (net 15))
 (segment (start 168.3997 119.2003) (end 176 111.6) (width 0.2) (layer "F.Cu") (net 15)))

